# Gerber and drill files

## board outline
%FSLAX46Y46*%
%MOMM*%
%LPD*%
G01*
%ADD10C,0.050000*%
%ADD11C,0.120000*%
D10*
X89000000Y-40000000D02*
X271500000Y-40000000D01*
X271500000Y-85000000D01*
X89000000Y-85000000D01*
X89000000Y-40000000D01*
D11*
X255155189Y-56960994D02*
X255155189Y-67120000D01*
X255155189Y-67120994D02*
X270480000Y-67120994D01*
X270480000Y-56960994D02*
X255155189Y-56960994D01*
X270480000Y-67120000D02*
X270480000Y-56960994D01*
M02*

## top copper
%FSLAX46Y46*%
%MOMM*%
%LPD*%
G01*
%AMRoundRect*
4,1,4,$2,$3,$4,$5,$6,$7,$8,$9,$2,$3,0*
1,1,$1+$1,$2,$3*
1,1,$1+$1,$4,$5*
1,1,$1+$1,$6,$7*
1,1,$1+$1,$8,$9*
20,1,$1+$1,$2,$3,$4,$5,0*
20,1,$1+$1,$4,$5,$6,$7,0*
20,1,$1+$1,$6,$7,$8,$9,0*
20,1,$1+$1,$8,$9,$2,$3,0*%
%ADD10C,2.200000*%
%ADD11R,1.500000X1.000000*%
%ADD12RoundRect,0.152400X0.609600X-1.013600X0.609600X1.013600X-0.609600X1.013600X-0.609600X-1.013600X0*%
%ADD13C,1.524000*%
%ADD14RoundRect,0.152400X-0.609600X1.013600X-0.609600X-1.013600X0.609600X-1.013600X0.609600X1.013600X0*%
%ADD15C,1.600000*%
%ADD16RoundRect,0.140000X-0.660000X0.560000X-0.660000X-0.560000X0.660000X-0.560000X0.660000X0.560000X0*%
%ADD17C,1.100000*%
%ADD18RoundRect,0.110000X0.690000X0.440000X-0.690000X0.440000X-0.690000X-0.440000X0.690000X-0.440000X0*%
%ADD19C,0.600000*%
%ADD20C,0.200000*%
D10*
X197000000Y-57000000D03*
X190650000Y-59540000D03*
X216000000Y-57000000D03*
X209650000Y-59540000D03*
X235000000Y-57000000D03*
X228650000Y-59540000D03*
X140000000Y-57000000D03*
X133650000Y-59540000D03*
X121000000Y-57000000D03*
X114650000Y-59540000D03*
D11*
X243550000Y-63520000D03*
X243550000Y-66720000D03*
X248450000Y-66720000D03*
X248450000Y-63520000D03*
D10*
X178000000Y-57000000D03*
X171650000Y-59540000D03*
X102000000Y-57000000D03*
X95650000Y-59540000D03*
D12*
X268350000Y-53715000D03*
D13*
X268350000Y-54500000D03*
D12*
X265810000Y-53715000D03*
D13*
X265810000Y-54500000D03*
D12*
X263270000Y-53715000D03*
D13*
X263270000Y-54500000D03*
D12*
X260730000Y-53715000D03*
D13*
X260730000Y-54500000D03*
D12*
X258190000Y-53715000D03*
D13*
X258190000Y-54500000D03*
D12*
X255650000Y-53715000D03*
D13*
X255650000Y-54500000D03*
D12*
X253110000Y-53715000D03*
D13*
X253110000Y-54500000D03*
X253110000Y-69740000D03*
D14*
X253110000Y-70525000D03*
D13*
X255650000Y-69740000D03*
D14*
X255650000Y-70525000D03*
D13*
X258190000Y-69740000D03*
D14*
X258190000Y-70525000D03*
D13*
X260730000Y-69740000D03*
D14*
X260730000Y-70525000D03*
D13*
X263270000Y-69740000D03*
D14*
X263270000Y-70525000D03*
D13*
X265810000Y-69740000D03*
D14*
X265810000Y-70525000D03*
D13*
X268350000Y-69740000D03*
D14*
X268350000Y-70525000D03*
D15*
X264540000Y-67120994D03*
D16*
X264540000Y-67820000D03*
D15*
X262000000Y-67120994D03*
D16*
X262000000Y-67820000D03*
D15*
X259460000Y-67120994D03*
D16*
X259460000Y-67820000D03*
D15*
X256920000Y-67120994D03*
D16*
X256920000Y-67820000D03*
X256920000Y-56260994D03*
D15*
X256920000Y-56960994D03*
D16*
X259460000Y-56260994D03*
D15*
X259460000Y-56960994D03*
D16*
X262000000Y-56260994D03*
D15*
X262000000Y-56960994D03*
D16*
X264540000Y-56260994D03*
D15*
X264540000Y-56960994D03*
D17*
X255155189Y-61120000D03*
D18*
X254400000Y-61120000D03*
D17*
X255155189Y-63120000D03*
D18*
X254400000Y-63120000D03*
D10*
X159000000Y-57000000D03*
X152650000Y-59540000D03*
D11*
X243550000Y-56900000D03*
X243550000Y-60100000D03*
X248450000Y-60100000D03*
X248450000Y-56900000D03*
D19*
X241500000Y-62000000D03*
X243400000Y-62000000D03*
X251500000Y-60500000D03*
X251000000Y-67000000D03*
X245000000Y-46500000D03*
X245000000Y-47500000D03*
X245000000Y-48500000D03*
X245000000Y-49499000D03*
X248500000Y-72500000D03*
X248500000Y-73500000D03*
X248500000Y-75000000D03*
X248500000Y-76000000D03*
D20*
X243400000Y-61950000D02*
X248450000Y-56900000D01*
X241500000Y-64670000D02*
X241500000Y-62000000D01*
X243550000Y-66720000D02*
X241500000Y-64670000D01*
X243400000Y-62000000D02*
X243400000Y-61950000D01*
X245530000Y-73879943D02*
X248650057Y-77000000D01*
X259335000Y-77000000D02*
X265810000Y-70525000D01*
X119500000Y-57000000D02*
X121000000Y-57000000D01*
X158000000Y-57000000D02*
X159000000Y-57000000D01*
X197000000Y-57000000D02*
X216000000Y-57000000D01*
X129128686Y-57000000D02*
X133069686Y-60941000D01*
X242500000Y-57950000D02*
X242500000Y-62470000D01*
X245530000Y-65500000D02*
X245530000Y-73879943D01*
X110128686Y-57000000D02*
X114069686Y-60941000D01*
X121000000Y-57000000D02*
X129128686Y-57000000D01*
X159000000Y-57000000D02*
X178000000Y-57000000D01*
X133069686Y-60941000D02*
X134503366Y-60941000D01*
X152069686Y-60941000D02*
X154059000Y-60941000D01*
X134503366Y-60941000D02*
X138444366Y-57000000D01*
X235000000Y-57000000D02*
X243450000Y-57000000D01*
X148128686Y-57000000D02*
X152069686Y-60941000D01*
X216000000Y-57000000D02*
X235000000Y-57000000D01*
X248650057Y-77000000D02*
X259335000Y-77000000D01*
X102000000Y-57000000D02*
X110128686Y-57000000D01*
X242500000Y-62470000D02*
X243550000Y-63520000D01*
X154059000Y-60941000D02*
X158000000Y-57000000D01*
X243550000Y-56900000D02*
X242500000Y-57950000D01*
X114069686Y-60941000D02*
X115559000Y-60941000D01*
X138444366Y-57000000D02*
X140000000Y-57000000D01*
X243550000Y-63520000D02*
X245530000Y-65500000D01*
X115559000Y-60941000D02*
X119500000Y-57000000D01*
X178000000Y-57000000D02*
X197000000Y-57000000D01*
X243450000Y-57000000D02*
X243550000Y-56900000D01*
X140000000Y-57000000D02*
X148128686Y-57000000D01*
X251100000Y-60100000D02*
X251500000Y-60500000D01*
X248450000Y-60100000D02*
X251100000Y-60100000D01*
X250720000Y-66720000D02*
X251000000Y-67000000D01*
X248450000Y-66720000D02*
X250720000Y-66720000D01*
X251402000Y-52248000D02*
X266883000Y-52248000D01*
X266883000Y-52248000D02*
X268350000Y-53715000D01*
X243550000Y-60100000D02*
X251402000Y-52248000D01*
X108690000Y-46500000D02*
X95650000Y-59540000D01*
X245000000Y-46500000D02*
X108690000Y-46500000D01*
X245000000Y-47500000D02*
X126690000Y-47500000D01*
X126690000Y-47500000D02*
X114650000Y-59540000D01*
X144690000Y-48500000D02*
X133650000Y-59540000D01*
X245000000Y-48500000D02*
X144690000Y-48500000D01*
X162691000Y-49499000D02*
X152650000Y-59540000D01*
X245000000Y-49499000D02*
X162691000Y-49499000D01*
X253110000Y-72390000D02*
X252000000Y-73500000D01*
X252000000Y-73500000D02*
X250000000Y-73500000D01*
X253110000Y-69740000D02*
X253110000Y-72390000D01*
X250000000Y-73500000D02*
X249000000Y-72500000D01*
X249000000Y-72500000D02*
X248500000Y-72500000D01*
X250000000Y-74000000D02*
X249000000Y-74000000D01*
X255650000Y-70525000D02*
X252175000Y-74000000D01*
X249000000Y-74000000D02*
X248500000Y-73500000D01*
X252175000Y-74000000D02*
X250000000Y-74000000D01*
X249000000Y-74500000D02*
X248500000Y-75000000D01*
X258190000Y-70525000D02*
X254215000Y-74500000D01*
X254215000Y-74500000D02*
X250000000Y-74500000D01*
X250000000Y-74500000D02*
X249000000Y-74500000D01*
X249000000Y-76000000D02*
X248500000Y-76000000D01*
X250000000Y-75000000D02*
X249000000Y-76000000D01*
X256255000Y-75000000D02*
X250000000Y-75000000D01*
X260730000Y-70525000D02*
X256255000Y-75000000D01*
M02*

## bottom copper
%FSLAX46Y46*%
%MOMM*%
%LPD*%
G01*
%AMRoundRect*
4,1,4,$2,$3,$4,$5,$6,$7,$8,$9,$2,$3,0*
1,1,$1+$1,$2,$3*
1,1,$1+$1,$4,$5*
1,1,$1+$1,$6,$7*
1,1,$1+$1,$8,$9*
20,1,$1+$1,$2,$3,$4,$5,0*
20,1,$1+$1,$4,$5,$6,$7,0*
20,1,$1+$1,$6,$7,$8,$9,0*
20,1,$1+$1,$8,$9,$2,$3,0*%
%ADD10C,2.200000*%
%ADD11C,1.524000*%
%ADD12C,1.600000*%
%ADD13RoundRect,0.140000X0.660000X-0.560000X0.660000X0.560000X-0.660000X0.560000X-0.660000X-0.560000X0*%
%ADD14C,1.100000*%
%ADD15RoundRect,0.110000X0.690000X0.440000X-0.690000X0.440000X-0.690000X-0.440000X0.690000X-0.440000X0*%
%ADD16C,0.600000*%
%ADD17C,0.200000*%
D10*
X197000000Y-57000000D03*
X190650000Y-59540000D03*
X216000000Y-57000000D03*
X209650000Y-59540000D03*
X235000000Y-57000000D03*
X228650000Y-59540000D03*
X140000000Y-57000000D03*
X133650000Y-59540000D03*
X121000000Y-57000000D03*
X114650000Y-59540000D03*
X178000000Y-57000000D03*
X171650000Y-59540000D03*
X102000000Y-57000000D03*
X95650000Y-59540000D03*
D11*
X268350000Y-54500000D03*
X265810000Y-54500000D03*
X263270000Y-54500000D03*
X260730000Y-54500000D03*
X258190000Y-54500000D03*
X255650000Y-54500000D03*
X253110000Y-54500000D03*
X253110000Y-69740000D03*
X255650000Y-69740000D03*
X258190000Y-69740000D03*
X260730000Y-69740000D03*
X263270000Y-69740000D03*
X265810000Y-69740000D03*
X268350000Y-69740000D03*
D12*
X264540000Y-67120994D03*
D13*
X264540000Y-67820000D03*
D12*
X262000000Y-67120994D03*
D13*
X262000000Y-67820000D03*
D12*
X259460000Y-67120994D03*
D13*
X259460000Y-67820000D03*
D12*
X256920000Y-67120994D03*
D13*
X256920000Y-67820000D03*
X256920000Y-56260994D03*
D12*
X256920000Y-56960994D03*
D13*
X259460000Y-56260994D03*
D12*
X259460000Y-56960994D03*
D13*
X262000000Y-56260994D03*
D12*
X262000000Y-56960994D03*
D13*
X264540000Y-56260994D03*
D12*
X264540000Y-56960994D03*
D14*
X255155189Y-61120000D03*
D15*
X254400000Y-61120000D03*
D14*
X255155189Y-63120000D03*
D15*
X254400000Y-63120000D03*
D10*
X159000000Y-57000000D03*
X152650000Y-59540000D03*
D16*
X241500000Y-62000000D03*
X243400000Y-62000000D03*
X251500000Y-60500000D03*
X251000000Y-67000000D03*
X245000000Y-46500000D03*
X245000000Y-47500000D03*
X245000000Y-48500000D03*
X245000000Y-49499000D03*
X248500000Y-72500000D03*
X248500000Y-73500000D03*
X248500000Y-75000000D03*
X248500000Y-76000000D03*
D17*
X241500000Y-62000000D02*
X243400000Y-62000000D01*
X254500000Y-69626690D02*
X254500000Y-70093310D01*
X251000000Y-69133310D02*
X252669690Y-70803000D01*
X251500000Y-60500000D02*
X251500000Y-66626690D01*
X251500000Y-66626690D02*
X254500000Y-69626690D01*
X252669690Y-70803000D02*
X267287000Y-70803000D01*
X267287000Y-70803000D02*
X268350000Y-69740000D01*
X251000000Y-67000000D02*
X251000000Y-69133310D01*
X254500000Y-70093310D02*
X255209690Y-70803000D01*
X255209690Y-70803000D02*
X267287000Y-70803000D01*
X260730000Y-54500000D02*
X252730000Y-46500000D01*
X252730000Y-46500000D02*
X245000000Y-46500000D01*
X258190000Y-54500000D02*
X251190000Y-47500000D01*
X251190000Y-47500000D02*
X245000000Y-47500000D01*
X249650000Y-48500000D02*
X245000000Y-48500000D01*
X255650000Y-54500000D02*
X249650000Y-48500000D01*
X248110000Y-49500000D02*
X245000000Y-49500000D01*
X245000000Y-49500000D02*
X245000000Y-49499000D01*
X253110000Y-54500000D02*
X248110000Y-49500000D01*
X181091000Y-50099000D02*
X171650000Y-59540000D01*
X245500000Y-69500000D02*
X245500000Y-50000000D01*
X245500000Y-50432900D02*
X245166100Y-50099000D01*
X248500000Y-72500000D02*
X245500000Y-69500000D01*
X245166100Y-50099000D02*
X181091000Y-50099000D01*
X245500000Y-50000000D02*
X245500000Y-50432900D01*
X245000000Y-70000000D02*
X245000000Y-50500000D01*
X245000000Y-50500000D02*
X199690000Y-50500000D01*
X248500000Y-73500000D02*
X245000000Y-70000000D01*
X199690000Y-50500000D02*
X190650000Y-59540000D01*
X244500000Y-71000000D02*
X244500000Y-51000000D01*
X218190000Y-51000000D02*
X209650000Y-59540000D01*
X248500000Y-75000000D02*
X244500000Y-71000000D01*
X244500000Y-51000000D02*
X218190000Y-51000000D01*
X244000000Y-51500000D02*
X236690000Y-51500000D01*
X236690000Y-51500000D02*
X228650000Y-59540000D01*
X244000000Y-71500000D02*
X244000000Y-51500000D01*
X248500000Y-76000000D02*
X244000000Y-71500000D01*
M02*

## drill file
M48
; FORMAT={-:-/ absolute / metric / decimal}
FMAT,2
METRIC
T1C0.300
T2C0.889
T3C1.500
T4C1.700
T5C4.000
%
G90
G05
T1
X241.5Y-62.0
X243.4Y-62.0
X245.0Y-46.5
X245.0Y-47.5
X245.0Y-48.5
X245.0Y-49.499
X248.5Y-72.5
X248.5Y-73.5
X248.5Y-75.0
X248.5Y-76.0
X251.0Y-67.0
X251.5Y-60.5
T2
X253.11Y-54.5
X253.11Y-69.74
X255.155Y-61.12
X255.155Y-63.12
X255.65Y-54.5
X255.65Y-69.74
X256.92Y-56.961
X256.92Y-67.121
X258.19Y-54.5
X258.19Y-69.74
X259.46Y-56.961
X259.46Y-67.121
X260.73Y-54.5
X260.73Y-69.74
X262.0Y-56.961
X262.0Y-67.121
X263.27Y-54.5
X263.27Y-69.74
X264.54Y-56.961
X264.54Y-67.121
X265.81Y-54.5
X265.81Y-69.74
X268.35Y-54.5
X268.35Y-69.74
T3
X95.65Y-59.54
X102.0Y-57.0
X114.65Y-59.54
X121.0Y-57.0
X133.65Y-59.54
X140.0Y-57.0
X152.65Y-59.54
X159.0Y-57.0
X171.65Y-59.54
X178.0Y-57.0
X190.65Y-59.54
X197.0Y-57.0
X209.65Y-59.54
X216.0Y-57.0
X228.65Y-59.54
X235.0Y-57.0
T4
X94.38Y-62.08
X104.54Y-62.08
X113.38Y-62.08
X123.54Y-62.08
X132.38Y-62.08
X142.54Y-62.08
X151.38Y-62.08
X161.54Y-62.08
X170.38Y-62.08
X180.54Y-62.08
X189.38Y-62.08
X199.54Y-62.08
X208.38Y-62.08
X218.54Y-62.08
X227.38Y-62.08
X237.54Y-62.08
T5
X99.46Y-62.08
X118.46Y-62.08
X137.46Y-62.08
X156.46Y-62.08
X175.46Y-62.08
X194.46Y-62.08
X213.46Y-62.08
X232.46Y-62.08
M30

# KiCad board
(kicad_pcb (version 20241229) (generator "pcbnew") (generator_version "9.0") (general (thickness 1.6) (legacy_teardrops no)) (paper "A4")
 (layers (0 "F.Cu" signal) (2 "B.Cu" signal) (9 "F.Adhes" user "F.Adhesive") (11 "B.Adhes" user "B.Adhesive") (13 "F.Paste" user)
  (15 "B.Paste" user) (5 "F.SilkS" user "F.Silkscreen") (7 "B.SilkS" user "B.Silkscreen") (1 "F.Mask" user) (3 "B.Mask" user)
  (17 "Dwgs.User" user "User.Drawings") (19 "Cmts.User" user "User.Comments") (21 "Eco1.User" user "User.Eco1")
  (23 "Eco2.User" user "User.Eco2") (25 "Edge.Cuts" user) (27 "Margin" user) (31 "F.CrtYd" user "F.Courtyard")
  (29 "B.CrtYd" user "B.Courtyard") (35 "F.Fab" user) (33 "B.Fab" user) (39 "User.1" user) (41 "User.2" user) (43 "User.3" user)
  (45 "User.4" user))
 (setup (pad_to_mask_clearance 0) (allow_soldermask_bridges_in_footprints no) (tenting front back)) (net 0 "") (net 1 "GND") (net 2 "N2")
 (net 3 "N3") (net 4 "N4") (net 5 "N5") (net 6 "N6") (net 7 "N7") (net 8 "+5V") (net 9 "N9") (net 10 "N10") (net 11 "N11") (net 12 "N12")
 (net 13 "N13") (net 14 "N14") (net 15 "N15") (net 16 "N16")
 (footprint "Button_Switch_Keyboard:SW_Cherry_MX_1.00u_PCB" (layer "F.Cu") (at 197 57)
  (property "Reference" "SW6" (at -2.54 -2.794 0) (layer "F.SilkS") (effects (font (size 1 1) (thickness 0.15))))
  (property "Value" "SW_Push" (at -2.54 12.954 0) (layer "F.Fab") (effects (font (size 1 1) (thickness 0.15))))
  (pad "" np_thru_hole circle (at -7.62 5.08) (size 1.7 1.7) (drill 1.7) (layers "*.Cu" "*.Mask"))
  (pad "" np_thru_hole circle (at -2.54 5.08) (size 4 4) (drill 4) (layers "*.Cu" "*.Mask"))
  (pad "" np_thru_hole circle (at 2.54 5.08) (size 1.7 1.7) (drill 1.7) (layers "*.Cu" "*.Mask"))
  (pad "1" thru_hole circle (at 0 0) (size 2.2 2.2) (drill 1.5) (layers "*.Cu" "*.Mask") (remove_unused_layers no) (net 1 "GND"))
  (pad "2" thru_hole circle (at -6.35 2.54) (size 2.2 2.2) (drill 1.5) (layers "*.Cu" "*.Mask") (remove_unused_layers no) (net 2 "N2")))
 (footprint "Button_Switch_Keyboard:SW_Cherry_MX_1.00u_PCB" (layer "F.Cu") (at 216 57)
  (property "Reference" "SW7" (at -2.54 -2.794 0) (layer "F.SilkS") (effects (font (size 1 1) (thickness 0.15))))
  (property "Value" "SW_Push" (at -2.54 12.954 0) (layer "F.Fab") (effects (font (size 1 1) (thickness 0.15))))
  (pad "" np_thru_hole circle (at -7.62 5.08) (size 1.7 1.7) (drill 1.7) (layers "*.Cu" "*.Mask"))
  (pad "" np_thru_hole circle (at -2.54 5.08) (size 4 4) (drill 4) (layers "*.Cu" "*.Mask"))
  (pad "" np_thru_hole circle (at 2.54 5.08) (size 1.7 1.7) (drill 1.7) (layers "*.Cu" "*.Mask"))
  (pad "1" thru_hole circle (at 0 0) (size 2.2 2.2) (drill 1.5) (layers "*.Cu" "*.Mask") (remove_unused_layers no) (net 1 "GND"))
  (pad "2" thru_hole circle (at -6.35 2.54) (size 2.2 2.2) (drill 1.5) (layers "*.Cu" "*.Mask") (remove_unused_layers no) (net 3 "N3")))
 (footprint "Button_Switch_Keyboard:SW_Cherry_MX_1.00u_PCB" (layer "F.Cu") (at 235 57)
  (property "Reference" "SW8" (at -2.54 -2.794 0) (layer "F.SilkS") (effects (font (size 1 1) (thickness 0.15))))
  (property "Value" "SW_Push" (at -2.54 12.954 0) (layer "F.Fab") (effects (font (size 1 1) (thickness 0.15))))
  (pad "" np_thru_hole circle (at -7.62 5.08) (size 1.7 1.7) (drill 1.7) (layers "*.Cu" "*.Mask"))
  (pad "" np_thru_hole circle (at -2.54 5.08) (size 4 4) (drill 4) (layers "*.Cu" "*.Mask"))
  (pad "" np_thru_hole circle (at 2.54 5.08) (size 1.7 1.7) (drill 1.7) (layers "*.Cu" "*.Mask"))
  (pad "1" thru_hole circle (at 0 0) (size 2.2 2.2) (drill 1.5) (layers "*.Cu" "*.Mask") (remove_unused_layers no) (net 1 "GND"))
  (pad "2" thru_hole circle (at -6.35 2.54) (size 2.2 2.2) (drill 1.5) (layers "*.Cu" "*.Mask") (remove_unused_layers no) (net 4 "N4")))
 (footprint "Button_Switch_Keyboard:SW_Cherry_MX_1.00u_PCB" (layer "F.Cu") (at 140 57)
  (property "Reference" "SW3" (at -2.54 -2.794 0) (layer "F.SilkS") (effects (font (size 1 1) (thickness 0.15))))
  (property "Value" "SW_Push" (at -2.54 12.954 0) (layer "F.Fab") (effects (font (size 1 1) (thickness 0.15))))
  (pad "" np_thru_hole circle (at -7.62 5.08) (size 1.7 1.7) (drill 1.7) (layers "*.Cu" "*.Mask"))
  (pad "" np_thru_hole circle (at -2.54 5.08) (size 4 4) (drill 4) (layers "*.Cu" "*.Mask"))
  (pad "" np_thru_hole circle (at 2.54 5.08) (size 1.7 1.7) (drill 1.7) (layers "*.Cu" "*.Mask"))
  (pad "1" thru_hole circle (at 0 0) (size 2.2 2.2) (drill 1.5) (layers "*.Cu" "*.Mask") (remove_unused_layers no) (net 1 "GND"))
  (pad "2" thru_hole circle (at -6.35 2.54) (size 2.2 2.2) (drill 1.5) (layers "*.Cu" "*.Mask") (remove_unused_layers no) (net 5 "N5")))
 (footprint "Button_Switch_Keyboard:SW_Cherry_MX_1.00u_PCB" (layer "F.Cu") (at 121 57)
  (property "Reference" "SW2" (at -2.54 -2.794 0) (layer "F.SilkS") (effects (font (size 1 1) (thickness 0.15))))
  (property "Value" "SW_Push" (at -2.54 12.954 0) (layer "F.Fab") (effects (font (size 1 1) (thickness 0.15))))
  (pad "" np_thru_hole circle (at -7.62 5.08) (size 1.7 1.7) (drill 1.7) (layers "*.Cu" "*.Mask"))
  (pad "" np_thru_hole circle (at -2.54 5.08) (size 4 4) (drill 4) (layers "*.Cu" "*.Mask"))
  (pad "" np_thru_hole circle (at 2.54 5.08) (size 1.7 1.7) (drill 1.7) (layers "*.Cu" "*.Mask"))
  (pad "1" thru_hole circle (at 0 0) (size 2.2 2.2) (drill 1.5) (layers "*.Cu" "*.Mask") (remove_unused_layers no) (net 1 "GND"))
  (pad "2" thru_hole circle (at -6.35 2.54) (size 2.2 2.2) (drill 1.5) (layers "*.Cu" "*.Mask") (remove_unused_layers no) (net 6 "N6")))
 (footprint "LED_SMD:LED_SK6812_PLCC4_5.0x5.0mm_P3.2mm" (layer "F.Cu") (at 246 65.12)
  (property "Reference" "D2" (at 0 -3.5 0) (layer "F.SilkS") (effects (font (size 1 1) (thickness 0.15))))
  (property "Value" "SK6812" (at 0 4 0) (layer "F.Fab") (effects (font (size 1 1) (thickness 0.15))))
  (pad "1" smd rect (at -2.45 -1.6 180) (size 1.5 1) (layers "F.Cu" "F.Mask" "F.Paste") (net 1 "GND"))
  (pad "2" smd rect (at -2.45 1.6 180) (size 1.5 1) (layers "F.Cu" "F.Mask" "F.Paste") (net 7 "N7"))
  (pad "3" smd rect (at 2.45 1.6 180) (size 1.5 1) (layers "F.Cu" "F.Mask" "F.Paste") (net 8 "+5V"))
  (pad "4" smd rect (at 2.45 -1.6 180) (size 1.5 1) (layers "F.Cu" "F.Mask" "F.Paste") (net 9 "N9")))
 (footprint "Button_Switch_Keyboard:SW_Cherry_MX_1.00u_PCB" (layer "F.Cu") (at 178 57)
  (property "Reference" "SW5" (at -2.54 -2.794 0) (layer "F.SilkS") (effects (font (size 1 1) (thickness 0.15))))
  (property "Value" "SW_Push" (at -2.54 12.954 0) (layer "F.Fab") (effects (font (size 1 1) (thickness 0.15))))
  (pad "" np_thru_hole circle (at -7.62 5.08) (size 1.7 1.7) (drill 1.7) (layers "*.Cu" "*.Mask"))
  (pad "" np_thru_hole circle (at -2.54 5.08) (size 4 4) (drill 4) (layers "*.Cu" "*.Mask"))
  (pad "" np_thru_hole circle (at 2.54 5.08) (size 1.7 1.7) (drill 1.7) (layers "*.Cu" "*.Mask"))
  (pad "1" thru_hole circle (at 0 0) (size 2.2 2.2) (drill 1.5) (layers "*.Cu" "*.Mask") (remove_unused_layers no) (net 1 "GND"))
  (pad "2" thru_hole circle (at -6.35 2.54) (size 2.2 2.2) (drill 1.5) (layers "*.Cu" "*.Mask") (remove_unused_layers no) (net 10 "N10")))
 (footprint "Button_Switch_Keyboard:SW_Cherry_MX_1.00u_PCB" (layer "F.Cu") (at 102 57)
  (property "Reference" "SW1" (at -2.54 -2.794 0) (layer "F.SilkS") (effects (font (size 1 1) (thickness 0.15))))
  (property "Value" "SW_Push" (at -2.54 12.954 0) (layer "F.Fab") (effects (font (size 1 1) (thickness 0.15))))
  (pad "" np_thru_hole circle (at -7.62 5.08) (size 1.7 1.7) (drill 1.7) (layers "*.Cu" "*.Mask"))
  (pad "" np_thru_hole circle (at -2.54 5.08) (size 4 4) (drill 4) (layers "*.Cu" "*.Mask"))
  (pad "" np_thru_hole circle (at 2.54 5.08) (size 1.7 1.7) (drill 1.7) (layers "*.Cu" "*.Mask"))
  (pad "1" thru_hole circle (at 0 0) (size 2.2 2.2) (drill 1.5) (layers "*.Cu" "*.Mask") (remove_unused_layers no) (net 1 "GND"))
  (pad "2" thru_hole circle (at -6.35 2.54) (size 2.2 2.2) (drill 1.5) (layers "*.Cu" "*.Mask") (remove_unused_layers no) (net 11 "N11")))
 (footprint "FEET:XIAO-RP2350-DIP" (layer "F.Cu") (at 260.7935 62.120994 -90)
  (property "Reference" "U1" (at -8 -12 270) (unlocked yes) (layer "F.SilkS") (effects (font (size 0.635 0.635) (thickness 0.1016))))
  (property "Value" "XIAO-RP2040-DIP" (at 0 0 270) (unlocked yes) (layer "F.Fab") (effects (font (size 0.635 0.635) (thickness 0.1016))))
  (fp_line (start -5.16 5.638311) (end 4.999006 5.638311) (stroke (width 0.12) (type default)) (layer "Edge.Cuts"))
  (fp_line (start 5 5.638311) (end 5 -9.6865) (stroke (width 0.12) (type default)) (layer "Edge.Cuts"))
  (fp_line (start -5.16 -9.6865) (end -5.16 5.638311) (stroke (width 0.12) (type default)) (layer "Edge.Cuts"))
  (fp_line (start 4.999006 -9.6865) (end -5.16 -9.6865) (stroke (width 0.12) (type default)) (layer "Edge.Cuts"))
  (pad "1" smd roundrect (at -8.405994 -7.5565 90) (size 2.332 1.524) (layers "F.Cu" "F.Mask") (roundrect_rratio 0.1) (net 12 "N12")
   (thermal_bridge_angle 45))
  (pad "1" thru_hole circle (at -7.620994 -7.5565 90) (size 1.524 1.524) (drill 0.889) (layers "*.Cu" "*.Mask") (remove_unused_layers no)
   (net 12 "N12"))
  (pad "2" smd roundrect (at -8.405994 -5.0165 90) (size 2.332 1.524) (layers "F.Cu" "F.Mask") (roundrect_rratio 0.1) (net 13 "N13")
   (thermal_bridge_angle 45))
  (pad "2" thru_hole circle (at -7.620994 -5.0165 90) (size 1.524 1.524) (drill 0.889) (layers "*.Cu" "*.Mask") (remove_unused_layers no)
   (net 13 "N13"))
  (pad "3" smd roundrect (at -8.405994 -2.4765 90) (size 2.332 1.524) (layers "F.Cu" "F.Mask") (roundrect_rratio 0.1) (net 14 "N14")
   (thermal_bridge_angle 45))
  (pad "3" thru_hole circle (at -7.620994 -2.4765 90) (size 1.524 1.524) (drill 0.889) (layers "*.Cu" "*.Mask") (remove_unused_layers no)
   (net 14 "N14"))
  (pad "4" smd roundrect (at -8.405994 0.0635 90) (size 2.332 1.524) (layers "F.Cu" "F.Mask") (roundrect_rratio 0.1) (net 11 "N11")
   (thermal_bridge_angle 45))
  (pad "4" thru_hole circle (at -7.620994 0.0635 90) (size 1.524 1.524) (drill 0.889) (layers "*.Cu" "*.Mask") (remove_unused_layers no)
   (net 11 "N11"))
  (pad "5" smd roundrect (at -8.405994 2.6035 90) (size 2.332 1.524) (layers "F.Cu" "F.Mask") (roundrect_rratio 0.1) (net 6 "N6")
   (thermal_bridge_angle 45))
  (pad "5" thru_hole circle (at -7.620994 2.6035 90) (size 1.524 1.524) (drill 0.889) (layers "*.Cu" "*.Mask") (remove_unused_layers no)
   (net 6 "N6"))
  (pad "6" smd roundrect (at -8.405994 5.1435 90) (size 2.332 1.524) (layers "F.Cu" "F.Mask") (roundrect_rratio 0.1) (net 5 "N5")
   (thermal_bridge_angle 45))
  (pad "6" thru_hole circle (at -7.620994 5.1435 90) (size 1.524 1.524) (drill 0.889) (layers "*.Cu" "*.Mask") (remove_unused_layers no)
   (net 5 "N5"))
  (pad "7" smd roundrect (at -8.405994 7.6835 90) (size 2.332 1.524) (layers "F.Cu" "F.Mask") (roundrect_rratio 0.1) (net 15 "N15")
   (thermal_bridge_angle 45))
  (pad "7" thru_hole circle (at -7.620994 7.6835 90) (size 1.524 1.524) (drill 0.889) (layers "*.Cu" "*.Mask") (remove_unused_layers no)
   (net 15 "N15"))
  (pad "8" thru_hole circle (at 7.619006 7.6835 270) (size 1.524 1.524) (drill 0.889) (layers "*.Cu" "*.Mask") (remove_unused_layers no)
   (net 10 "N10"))
  (pad "8" smd roundrect (at 8.404006 7.6835 270) (size 2.332 1.524) (layers "F.Cu" "F.Mask") (roundrect_rratio 0.1) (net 10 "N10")
   (thermal_bridge_angle 45))
  (pad "9" thru_hole circle (at 7.619006 5.1435 270) (size 1.524 1.524) (drill 0.889) (layers "*.Cu" "*.Mask") (remove_unused_layers no)
   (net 2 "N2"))
  (pad "9" smd roundrect (at 8.404006 5.1435 270) (size 2.332 1.524) (layers "F.Cu" "F.Mask") (roundrect_rratio 0.1) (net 2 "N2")
   (thermal_bridge_angle 45))
  (pad "10" thru_hole circle (at 7.619006 2.6035 270) (size 1.524 1.524) (drill 0.889) (layers "*.Cu" "*.Mask") (remove_unused_layers no)
   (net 3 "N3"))
  (pad "10" smd roundrect (at 8.404006 2.6035 270) (size 2.332 1.524) (layers "F.Cu" "F.Mask") (roundrect_rratio 0.1) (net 3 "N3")
   (thermal_bridge_angle 45))
  (pad "11" thru_hole circle (at 7.619006 0.0635 270) (size 1.524 1.524) (drill 0.889) (layers "*.Cu" "*.Mask") (remove_unused_layers no)
   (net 4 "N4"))
  (pad "11" smd roundrect (at 8.404006 0.0635 270) (size 2.332 1.524) (layers "F.Cu" "F.Mask") (roundrect_rratio 0.1) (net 4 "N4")
   (thermal_bridge_angle 45))
  (pad "12" thru_hole circle (at 7.619006 -2.4765 270) (size 1.524 1.524) (drill 0.889) (layers "*.Cu" "*.Mask") (remove_unused_layers no)
   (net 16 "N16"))
  (pad "12" smd roundrect (at 8.404006 -2.4765 270) (size 2.332 1.524) (layers "F.Cu" "F.Mask") (roundrect_rratio 0.1) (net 16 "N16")
   (thermal_bridge_angle 45))
  (pad "13" thru_hole circle (at 7.619006 -5.0165 270) (size 1.524 1.524) (drill 0.889) (layers "*.Cu" "*.Mask") (remove_unused_layers no)
   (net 1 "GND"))
  (pad "13" smd roundrect (at 8.404006 -5.0165 270) (size 2.332 1.524) (layers "F.Cu" "F.Mask") (roundrect_rratio 0.1) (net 1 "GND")
   (thermal_bridge_angle 45))
  (pad "14" thru_hole circle (at 7.619006 -7.5565 270) (size 1.524 1.524) (drill 0.889) (layers "*.Cu" "*.Mask") (remove_unused_layers no)
   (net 8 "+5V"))
  (pad "14" smd roundrect (at 8.404006 -7.5565 270) (size 2.332 1.524) (layers "F.Cu" "F.Mask") (roundrect_rratio 0.1) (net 8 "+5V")
   (thermal_bridge_angle 45))
  (pad "15" thru_hole circle (at 5 -3.7465 90) (size 1.6 1.6) (drill 0.889) (layers "*.Cu" "*.Mask") (remove_unused_layers no))
  (pad "15" smd roundrect (at 5.699006 -3.7465 270) (size 1.4 1.6) (layers "F.Cu" "F.Mask") (roundrect_rratio 0.1) (thermal_bridge_angle 45))
  (pad "15" smd roundrect (at 5.699006 -3.7465 90) (size 1.4 1.6) (layers "B.Cu" "B.Mask" "B.Paste") (roundrect_rratio 0.1)
   (thermal_bridge_angle 45))
  (pad "16" thru_hole circle (at 5 -1.2065 90) (size 1.6 1.6) (drill 0.889) (layers "*.Cu" "*.Mask") (remove_unused_layers no))
  (pad "16" smd roundrect (at 5.699006 -1.2065 270) (size 1.4 1.6) (layers "F.Cu" "F.Mask") (roundrect_rratio 0.1) (thermal_bridge_angle 45))
  (pad "16" smd roundrect (at 5.699006 -1.2065 90) (size 1.4 1.6) (layers "B.Cu" "B.Mask" "B.Paste") (roundrect_rratio 0.1)
   (thermal_bridge_angle 45))
  (pad "17" thru_hole circle (at 5 1.3335 90) (size 1.6 1.6) (drill 0.889) (layers "*.Cu" "*.Mask") (remove_unused_layers no))
  (pad "17" smd roundrect (at 5.699006 1.3335 270) (size 1.4 1.6) (layers "F.Cu" "F.Mask") (roundrect_rratio 0.1) (thermal_bridge_angle 45))
  (pad "17" smd roundrect (at 5.699006 1.3335 90) (size 1.4 1.6) (layers "B.Cu" "B.Mask" "B.Paste") (roundrect_rratio 0.1)
   (thermal_bridge_angle 45))
  (pad "18" thru_hole circle (at 5 3.8735 90) (size 1.6 1.6) (drill 0.889) (layers "*.Cu" "*.Mask") (remove_unused_layers no))
  (pad "18" smd roundrect (at 5.699006 3.8735 270) (size 1.4 1.6) (layers "F.Cu" "F.Mask") (roundrect_rratio 0.1) (thermal_bridge_angle 45))
  (pad "18" smd roundrect (at 5.699006 3.8735 90) (size 1.4 1.6) (layers "B.Cu" "B.Mask" "B.Paste") (roundrect_rratio 0.1)
   (thermal_bridge_angle 45))
  (pad "19" smd roundrect (at -5.86 3.8735 270) (size 1.4 1.6) (layers "F.Cu" "F.Mask") (roundrect_rratio 0.1) (thermal_bridge_angle 45))
  (pad "19" smd roundrect (at -5.86 3.8735 90) (size 1.4 1.6) (layers "B.Cu" "B.Mask" "B.Paste") (roundrect_rratio 0.1)
   (thermal_bridge_angle 45))
  (pad "19" thru_hole circle (at -5.16 3.8735 90) (size 1.6 1.6) (drill 0.889) (layers "*.Cu" "*.Mask") (remove_unused_layers no))
  (pad "20" smd roundrect (at -5.86 1.3335 270) (size 1.4 1.6) (layers "F.Cu" "F.Mask") (roundrect_rratio 0.1) (thermal_bridge_angle 45))
  (pad "20" smd roundrect (at -5.86 1.3335 90) (size 1.4 1.6) (layers "B.Cu" "B.Mask" "B.Paste") (roundrect_rratio 0.1)
   (thermal_bridge_angle 45))
  (pad "20" thru_hole circle (at -5.16 1.3335 90) (size 1.6 1.6) (drill 0.889) (layers "*.Cu" "*.Mask") (remove_unused_layers no))
  (pad "21" smd roundrect (at -5.86 -1.2065 270) (size 1.4 1.6) (layers "F.Cu" "F.Mask") (roundrect_rratio 0.1) (thermal_bridge_angle 45))
  (pad "21" smd roundrect (at -5.86 -1.2065 90) (size 1.4 1.6) (layers "B.Cu" "B.Mask" "B.Paste") (roundrect_rratio 0.1)
   (thermal_bridge_angle 45))
  (pad "21" thru_hole circle (at -5.16 -1.2065 90) (size 1.6 1.6) (drill 0.889) (layers "*.Cu" "*.Mask") (remove_unused_layers no))
  (pad "22" smd roundrect (at -5.86 -3.7465 270) (size 1.4 1.6) (layers "F.Cu" "F.Mask") (roundrect_rratio 0.1) (thermal_bridge_angle 45))
  (pad "22" smd roundrect (at -5.86 -3.7465 90) (size 1.4 1.6) (layers "B.Cu" "B.Mask" "B.Paste") (roundrect_rratio 0.1)
   (thermal_bridge_angle 45))
  (pad "22" thru_hole circle (at -5.16 -3.7465 90) (size 1.6 1.6) (drill 0.889) (layers "*.Cu" "*.Mask") (remove_unused_layers no))
  (pad "23" thru_hole circle (at -1.000994 5.638311 90) (size 1.1 1.1) (drill 0.889) (layers "*.Cu" "*.Mask") (remove_unused_layers no))
  (pad "23" smd roundrect (at -1.000994 6.3935 180) (size 1.6 1.1) (layers "F.Cu" "F.Mask") (roundrect_rratio 0.1) (thermal_bridge_angle 45))
  (pad "23" smd roundrect (at -1.000994 6.3935 180) (size 1.6 1.1) (layers "B.Cu" "B.Mask" "B.Paste") (roundrect_rratio 0.1)
   (thermal_bridge_angle 45))
  (pad "24" thru_hole circle (at 0.999006 5.638311 90) (size 1.1 1.1) (drill 0.889) (layers "*.Cu" "*.Mask") (remove_unused_layers no))
  (pad "24" smd roundrect (at 0.999006 6.3935 180) (size 1.6 1.1) (layers "F.Cu" "F.Mask") (roundrect_rratio 0.1) (thermal_bridge_angle 45))
  (pad "24" smd roundrect (at 0.999006 6.3935 180) (size 1.6 1.1) (layers "B.Cu" "B.Mask" "B.Paste") (roundrect_rratio 0.1)
   (thermal_bridge_angle 45)))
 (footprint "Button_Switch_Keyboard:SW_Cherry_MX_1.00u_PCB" (layer "F.Cu") (at 159 57)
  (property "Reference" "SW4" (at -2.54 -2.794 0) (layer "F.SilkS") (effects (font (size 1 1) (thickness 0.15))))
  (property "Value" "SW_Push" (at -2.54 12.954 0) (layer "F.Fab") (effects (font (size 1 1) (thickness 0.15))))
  (pad "" np_thru_hole circle (at -7.62 5.08) (size 1.7 1.7) (drill 1.7) (layers "*.Cu" "*.Mask"))
  (pad "" np_thru_hole circle (at -2.54 5.08) (size 4 4) (drill 4) (layers "*.Cu" "*.Mask"))
  (pad "" np_thru_hole circle (at 2.54 5.08) (size 1.7 1.7) (drill 1.7) (layers "*.Cu" "*.Mask"))
  (pad "1" thru_hole circle (at 0 0) (size 2.2 2.2) (drill 1.5) (layers "*.Cu" "*.Mask") (remove_unused_layers no) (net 1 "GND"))
  (pad "2" thru_hole circle (at -6.35 2.54) (size 2.2 2.2) (drill 1.5) (layers "*.Cu" "*.Mask") (remove_unused_layers no) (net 15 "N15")))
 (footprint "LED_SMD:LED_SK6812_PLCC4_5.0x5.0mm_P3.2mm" (layer "F.Cu") (at 246 58.5)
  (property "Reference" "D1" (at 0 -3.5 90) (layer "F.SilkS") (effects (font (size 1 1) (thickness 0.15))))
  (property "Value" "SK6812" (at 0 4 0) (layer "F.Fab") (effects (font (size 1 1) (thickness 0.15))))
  (pad "1" smd rect (at -2.45 -1.6 180) (size 1.5 1) (layers "F.Cu" "F.Mask" "F.Paste") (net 1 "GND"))
  (pad "2" smd rect (at -2.45 1.6 180) (size 1.5 1) (layers "F.Cu" "F.Mask" "F.Paste") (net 12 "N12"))
  (pad "3" smd rect (at 2.45 1.6 180) (size 1.5 1) (layers "F.Cu" "F.Mask" "F.Paste") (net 8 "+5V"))
  (pad "4" smd rect (at 2.45 -1.6 180) (size 1.5 1) (layers "F.Cu" "F.Mask" "F.Paste") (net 7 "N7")))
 (gr_rect (start 89 40) (end 271.5 85) (stroke (width 0.05) (type default)) (fill no) (layer "Edge.Cuts"))
 (segment (start 243.4 61.95) (end 248.45 56.9) (width 0.2) (layer "F.Cu") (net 7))
 (segment (start 241.5 64.67) (end 241.5 62) (width 0.2) (layer "F.Cu") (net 7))
 (segment (start 243.55 66.72) (end 241.5 64.67) (width 0.2) (layer "F.Cu") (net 7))
 (segment (start 243.4 62) (end 243.4 61.95) (width 0.2) (layer "F.Cu") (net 7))
 (via (at 241.5 62) (size 0.6) (drill 0.3) (layers "F.Cu" "B.Cu") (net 7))
 (via (at 243.4 62) (size 0.6) (drill 0.3) (layers "F.Cu" "B.Cu") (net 7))
 (segment (start 241.5 62) (end 243.4 62) (width 0.2) (layer "B.Cu") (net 7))
 (segment (start 245.53 73.879943) (end 248.650057 77) (width 0.2) (layer "F.Cu") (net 1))
 (segment (start 259.335 77) (end 265.81 70.525) (width 0.2) (layer "F.Cu") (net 1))
 (segment (start 119.5 57) (end 121 57) (width 0.2) (layer "F.Cu") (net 1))
 (segment (start 158 57) (end 159 57) (width 0.2) (layer "F.Cu") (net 1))
 (segment (start 197 57) (end 216 57) (width 0.2) (layer "F.Cu") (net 1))
 (segment (start 129.128686 57) (end 133.069686 60.941) (width 0.2) (layer "F.Cu") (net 1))
 (segment (start 242.5 57.95) (end 242.5 62.47) (width 0.2) (layer "F.Cu") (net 1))
 (segment (start 245.53 65.5) (end 245.53 73.879943) (width 0.2) (layer "F.Cu") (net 1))
 (segment (start 110.128686 57) (end 114.069686 60.941) (width 0.2) (layer "F.Cu") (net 1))
 (segment (start 121 57) (end 129.128686 57) (width 0.2) (layer "F.Cu") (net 1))
 (segment (start 159 57) (end 178 57) (width 0.2) (layer "F.Cu") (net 1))
 (segment (start 133.069686 60.941) (end 134.503366 60.941) (width 0.2) (layer "F.Cu") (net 1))
 (segment (start 152.069686 60.941) (end 154.059 60.941) (width 0.2) (layer "F.Cu") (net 1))
 (segment (start 134.503366 60.941) (end 138.444366 57) (width 0.2) (layer "F.Cu") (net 1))
 (segment (start 235 57) (end 243.45 57) (width 0.2) (layer "F.Cu") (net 1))
 (segment (start 148.128686 57) (end 152.069686 60.941) (width 0.2) (layer "F.Cu") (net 1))
 (segment (start 216 57) (end 235 57) (width 0.2) (layer "F.Cu") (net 1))
 (segment (start 248.650057 77) (end 259.335 77) (width 0.2) (layer "F.Cu") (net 1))
 (segment (start 102 57) (end 110.128686 57) (width 0.2) (layer "F.Cu") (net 1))
 (segment (start 242.5 62.47) (end 243.55 63.52) (width 0.2) (layer "F.Cu") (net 1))
 (segment (start 154.059 60.941) (end 158 57) (width 0.2) (layer "F.Cu") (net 1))
 (segment (start 243.55 56.9) (end 242.5 57.95) (width 0.2) (layer "F.Cu") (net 1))
 (segment (start 114.069686 60.941) (end 115.559 60.941) (width 0.2) (layer "F.Cu") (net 1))
 (segment (start 138.444366 57) (end 140 57) (width 0.2) (layer "F.Cu") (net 1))
 (segment (start 243.55 63.52) (end 245.53 65.5) (width 0.2) (layer "F.Cu") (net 1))
 (segment (start 115.559 60.941) (end 119.5 57) (width 0.2) (layer "F.Cu") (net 1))
 (segment (start 178 57) (end 197 57) (width 0.2) (layer "F.Cu") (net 1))
 (segment (start 243.45 57) (end 243.55 56.9) (width 0.2) (layer "F.Cu") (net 1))
 (segment (start 140 57) (end 148.128686 57) (width 0.2) (layer "F.Cu") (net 1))
 (segment (start 251.1 60.1) (end 251.5 60.5) (width 0.2) (layer "F.Cu") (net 8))
 (segment (start 248.45 60.1) (end 251.1 60.1) (width 0.2) (layer "F.Cu") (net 8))
 (segment (start 250.72 66.72) (end 251 67) (width 0.2) (layer "F.Cu") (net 8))
 (segment (start 248.45 66.72) (end 250.72 66.72) (width 0.2) (layer "F.Cu") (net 8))
 (via (at 251.5 60.5) (size 0.6) (drill 0.3) (layers "F.Cu" "B.Cu") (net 8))
 (via (at 251 67) (size 0.6) (drill 0.3) (layers "F.Cu" "B.Cu") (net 8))
 (segment (start 254.5 69.62669) (end 254.5 70.09331) (width 0.2) (layer "B.Cu") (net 8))
 (segment (start 251 69.13331) (end 252.66969 70.803) (width 0.2) (layer "B.Cu") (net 8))
 (segment (start 251.5 60.5) (end 251.5 66.62669) (width 0.2) (layer "B.Cu") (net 8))
 (segment (start 251.5 66.62669) (end 254.5 69.62669) (width 0.2) (layer "B.Cu") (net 8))
 (segment (start 252.66969 70.803) (end 267.287 70.803) (width 0.2) (layer "B.Cu") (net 8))
 (segment (start 267.287 70.803) (end 268.35 69.74) (width 0.2) (layer "B.Cu") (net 8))
 (segment (start 251 67) (end 251 69.13331) (width 0.2) (layer "B.Cu") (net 8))
 (segment (start 254.5 70.09331) (end 255.20969 70.803) (width 0.2) (layer "B.Cu") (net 8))
 (segment (start 255.20969 70.803) (end 267.287 70.803) (width 0.2) (layer "B.Cu") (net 8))
 (segment (start 251.402 52.248) (end 266.883 52.248) (width 0.2) (layer "F.Cu") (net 12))
 (segment (start 266.883 52.248) (end 268.35 53.715) (width 0.2) (layer "F.Cu") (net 12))
 (segment (start 243.55 60.1) (end 251.402 52.248) (width 0.2) (layer "F.Cu") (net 12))
 (segment (start 108.69 46.5) (end 95.65 59.54) (width 0.2) (layer "F.Cu") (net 11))
 (segment (start 245 46.5) (end 108.69 46.5) (width 0.2) (layer "F.Cu") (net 11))
 (via (at 245 46.5) (size 0.6) (drill 0.3) (layers "F.Cu" "B.Cu") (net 11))
 (segment (start 260.73 54.5) (end 252.73 46.5) (width 0.2) (layer "B.Cu") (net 11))
 (segment (start 252.73 46.5) (end 245 46.5) (width 0.2) (layer "B.Cu") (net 11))
 (segment (start 245 47.5) (end 126.69 47.5) (width 0.2) (layer "F.Cu") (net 6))
 (segment (start 126.69 47.5) (end 114.65 59.54) (width 0.2) (layer "F.Cu") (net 6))
 (via (at 245 47.5) (size 0.6) (drill 0.3) (layers "F.Cu" "B.Cu") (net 6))
 (segment (start 258.19 54.5) (end 251.19 47.5) (width 0.2) (layer "B.Cu") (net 6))
 (segment (start 251.19 47.5) (end 245 47.5) (width 0.2) (layer "B.Cu") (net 6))
 (segment (start 144.69 48.5) (end 133.65 59.54) (width 0.2) (layer "F.Cu") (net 5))
 (segment (start 245 48.5) (end 144.69 48.5) (width 0.2) (layer "F.Cu") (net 5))
 (via (at 245 48.5) (size 0.6) (drill 0.3) (layers "F.Cu" "B.Cu") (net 5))
 (segment (start 249.65 48.5) (end 245 48.5) (width 0.2) (layer "B.Cu") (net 5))
 (segment (start 255.65 54.5) (end 249.65 48.5) (width 0.2) (layer "B.Cu") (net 5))
 (segment (start 162.691 49.499) (end 152.65 59.54) (width 0.2) (layer "F.Cu") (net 15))
 (segment (start 245 49.499) (end 162.691 49.499) (width 0.2) (layer "F.Cu") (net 15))
 (via (at 245 49.499) (size 0.6) (drill 0.3) (layers "F.Cu" "B.Cu") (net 15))
 (segment (start 248.11 49.5) (end 245 49.5) (width 0.2) (layer "B.Cu") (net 15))
 (segment (start 245 49.5) (end 245 49.499) (width 0.2) (layer "B.Cu") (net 15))
 (segment (start 253.11 54.5) (end 248.11 49.5) (width 0.2) (layer "B.Cu") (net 15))
 (segment (start 253.11 72.39) (end 252 73.5) (width 0.2) (layer "F.Cu") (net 10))
 (segment (start 252 73.5) (end 250 73.5) (width 0.2) (layer "F.Cu") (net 10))
 (segment (start 253.11 69.74) (end 253.11 72.39) (width 0.2) (layer "F.Cu") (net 10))
 (segment (start 250 73.5) (end 249 72.5) (width 0.2) (layer "F.Cu") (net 10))
 (segment (start 249 72.5) (end 248.5 72.5) (width 0.2) (layer "F.Cu") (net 10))
 (via (at 248.5 72.5) (size 0.6) (drill 0.3) (layers "F.Cu" "B.Cu") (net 10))
 (segment (start 181.091 50.099) (end 171.65 59.54) (width 0.2) (layer "B.Cu") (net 10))
 (segment (start 245.5 69.5) (end 245.5 50) (width 0.2) (layer "B.Cu") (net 10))
 (segment (start 245.5 50.4329) (end 245.1661 50.099) (width 0.2) (layer "B.Cu") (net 10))
 (segment (start 248.5 72.5) (end 245.5 69.5) (width 0.2) (layer "B.Cu") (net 10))
 (segment (start 245.1661 50.099) (end 181.091 50.099) (width 0.2) (layer "B.Cu") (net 10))
 (segment (start 245.5 50) (end 245.5 50.4329) (width 0.2) (layer "B.Cu") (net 10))
 (segment (start 250 74) (end 249 74) (width 0.2) (layer "F.Cu") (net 2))
 (segment (start 255.65 70.525) (end 252.175 74) (width 0.2) (layer "F.Cu") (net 2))
 (segment (start 249 74) (end 248.5 73.5) (width 0.2) (layer "F.Cu") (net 2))
 (segment (start 252.175 74) (end 250 74) (width 0.2) (layer "F.Cu") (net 2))
 (via (at 248.5 73.5) (size 0.6) (drill 0.3) (layers "F.Cu" "B.Cu") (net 2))
 (segment (start 245 70) (end 245 50.5) (width 0.2) (layer "B.Cu") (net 2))
 (segment (start 245 50.5) (end 199.69 50.5) (width 0.2) (layer "B.Cu") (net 2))
 (segment (start 248.5 73.5) (end 245 70) (width 0.2) (layer "B.Cu") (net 2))
 (segment (start 199.69 50.5) (end 190.65 59.54) (width 0.2) (layer "B.Cu") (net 2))
 (segment (start 249 74.5) (end 248.5 75) (width 0.2) (layer "F.Cu") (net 3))
 (segment (start 258.19 70.525) (end 254.215 74.5) (width 0.2) (layer "F.Cu") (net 3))
 (segment (start 254.215 74.5) (end 250 74.5) (width 0.2) (layer "F.Cu") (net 3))
 (segment (start 250 74.5) (end 249 74.5) (width 0.2) (layer "F.Cu") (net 3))
 (via (at 248.5 75) (size 0.6) (drill 0.3) (layers "F.Cu" "B.Cu") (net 3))
 (segment (start 244.5 71) (end 244.5 51) (width 0.2) (layer "B.Cu") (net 3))
 (segment (start 218.19 51) (end 209.65 59.54) (width 0.2) (layer "B.Cu") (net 3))
 (segment (start 248.5 75) (end 244.5 71) (width 0.2) (layer "B.Cu") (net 3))
 (segment (start 244.5 51) (end 218.19 51) (width 0.2) (layer "B.Cu") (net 3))
 (segment (start 249 76) (end 248.5 76) (width 0.2) (layer "F.Cu") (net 4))
 (segment (start 250 75) (end 249 76) (width 0.2) (layer "F.Cu") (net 4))
 (segment (start 256.255 75) (end 250 75) (width 0.2) (layer "F.Cu") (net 4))
 (segment (start 260.73 70.525) (end 256.255 75) (width 0.2) (layer "F.Cu") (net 4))
 (via (at 248.5 76) (size 0.6) (drill 0.3) (layers "F.Cu" "B.Cu") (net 4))
 (segment (start 244 51.5) (end 236.69 51.5) (width 0.2) (layer "B.Cu") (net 4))
 (segment (start 236.69 51.5) (end 228.65 59.54) (width 0.2) (layer "B.Cu") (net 4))
 (segment (start 244 71.5) (end 244 51.5) (width 0.2) (layer "B.Cu") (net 4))
 (segment (start 248.5 76) (end 244 71.5) (width 0.2) (layer "B.Cu") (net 4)))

